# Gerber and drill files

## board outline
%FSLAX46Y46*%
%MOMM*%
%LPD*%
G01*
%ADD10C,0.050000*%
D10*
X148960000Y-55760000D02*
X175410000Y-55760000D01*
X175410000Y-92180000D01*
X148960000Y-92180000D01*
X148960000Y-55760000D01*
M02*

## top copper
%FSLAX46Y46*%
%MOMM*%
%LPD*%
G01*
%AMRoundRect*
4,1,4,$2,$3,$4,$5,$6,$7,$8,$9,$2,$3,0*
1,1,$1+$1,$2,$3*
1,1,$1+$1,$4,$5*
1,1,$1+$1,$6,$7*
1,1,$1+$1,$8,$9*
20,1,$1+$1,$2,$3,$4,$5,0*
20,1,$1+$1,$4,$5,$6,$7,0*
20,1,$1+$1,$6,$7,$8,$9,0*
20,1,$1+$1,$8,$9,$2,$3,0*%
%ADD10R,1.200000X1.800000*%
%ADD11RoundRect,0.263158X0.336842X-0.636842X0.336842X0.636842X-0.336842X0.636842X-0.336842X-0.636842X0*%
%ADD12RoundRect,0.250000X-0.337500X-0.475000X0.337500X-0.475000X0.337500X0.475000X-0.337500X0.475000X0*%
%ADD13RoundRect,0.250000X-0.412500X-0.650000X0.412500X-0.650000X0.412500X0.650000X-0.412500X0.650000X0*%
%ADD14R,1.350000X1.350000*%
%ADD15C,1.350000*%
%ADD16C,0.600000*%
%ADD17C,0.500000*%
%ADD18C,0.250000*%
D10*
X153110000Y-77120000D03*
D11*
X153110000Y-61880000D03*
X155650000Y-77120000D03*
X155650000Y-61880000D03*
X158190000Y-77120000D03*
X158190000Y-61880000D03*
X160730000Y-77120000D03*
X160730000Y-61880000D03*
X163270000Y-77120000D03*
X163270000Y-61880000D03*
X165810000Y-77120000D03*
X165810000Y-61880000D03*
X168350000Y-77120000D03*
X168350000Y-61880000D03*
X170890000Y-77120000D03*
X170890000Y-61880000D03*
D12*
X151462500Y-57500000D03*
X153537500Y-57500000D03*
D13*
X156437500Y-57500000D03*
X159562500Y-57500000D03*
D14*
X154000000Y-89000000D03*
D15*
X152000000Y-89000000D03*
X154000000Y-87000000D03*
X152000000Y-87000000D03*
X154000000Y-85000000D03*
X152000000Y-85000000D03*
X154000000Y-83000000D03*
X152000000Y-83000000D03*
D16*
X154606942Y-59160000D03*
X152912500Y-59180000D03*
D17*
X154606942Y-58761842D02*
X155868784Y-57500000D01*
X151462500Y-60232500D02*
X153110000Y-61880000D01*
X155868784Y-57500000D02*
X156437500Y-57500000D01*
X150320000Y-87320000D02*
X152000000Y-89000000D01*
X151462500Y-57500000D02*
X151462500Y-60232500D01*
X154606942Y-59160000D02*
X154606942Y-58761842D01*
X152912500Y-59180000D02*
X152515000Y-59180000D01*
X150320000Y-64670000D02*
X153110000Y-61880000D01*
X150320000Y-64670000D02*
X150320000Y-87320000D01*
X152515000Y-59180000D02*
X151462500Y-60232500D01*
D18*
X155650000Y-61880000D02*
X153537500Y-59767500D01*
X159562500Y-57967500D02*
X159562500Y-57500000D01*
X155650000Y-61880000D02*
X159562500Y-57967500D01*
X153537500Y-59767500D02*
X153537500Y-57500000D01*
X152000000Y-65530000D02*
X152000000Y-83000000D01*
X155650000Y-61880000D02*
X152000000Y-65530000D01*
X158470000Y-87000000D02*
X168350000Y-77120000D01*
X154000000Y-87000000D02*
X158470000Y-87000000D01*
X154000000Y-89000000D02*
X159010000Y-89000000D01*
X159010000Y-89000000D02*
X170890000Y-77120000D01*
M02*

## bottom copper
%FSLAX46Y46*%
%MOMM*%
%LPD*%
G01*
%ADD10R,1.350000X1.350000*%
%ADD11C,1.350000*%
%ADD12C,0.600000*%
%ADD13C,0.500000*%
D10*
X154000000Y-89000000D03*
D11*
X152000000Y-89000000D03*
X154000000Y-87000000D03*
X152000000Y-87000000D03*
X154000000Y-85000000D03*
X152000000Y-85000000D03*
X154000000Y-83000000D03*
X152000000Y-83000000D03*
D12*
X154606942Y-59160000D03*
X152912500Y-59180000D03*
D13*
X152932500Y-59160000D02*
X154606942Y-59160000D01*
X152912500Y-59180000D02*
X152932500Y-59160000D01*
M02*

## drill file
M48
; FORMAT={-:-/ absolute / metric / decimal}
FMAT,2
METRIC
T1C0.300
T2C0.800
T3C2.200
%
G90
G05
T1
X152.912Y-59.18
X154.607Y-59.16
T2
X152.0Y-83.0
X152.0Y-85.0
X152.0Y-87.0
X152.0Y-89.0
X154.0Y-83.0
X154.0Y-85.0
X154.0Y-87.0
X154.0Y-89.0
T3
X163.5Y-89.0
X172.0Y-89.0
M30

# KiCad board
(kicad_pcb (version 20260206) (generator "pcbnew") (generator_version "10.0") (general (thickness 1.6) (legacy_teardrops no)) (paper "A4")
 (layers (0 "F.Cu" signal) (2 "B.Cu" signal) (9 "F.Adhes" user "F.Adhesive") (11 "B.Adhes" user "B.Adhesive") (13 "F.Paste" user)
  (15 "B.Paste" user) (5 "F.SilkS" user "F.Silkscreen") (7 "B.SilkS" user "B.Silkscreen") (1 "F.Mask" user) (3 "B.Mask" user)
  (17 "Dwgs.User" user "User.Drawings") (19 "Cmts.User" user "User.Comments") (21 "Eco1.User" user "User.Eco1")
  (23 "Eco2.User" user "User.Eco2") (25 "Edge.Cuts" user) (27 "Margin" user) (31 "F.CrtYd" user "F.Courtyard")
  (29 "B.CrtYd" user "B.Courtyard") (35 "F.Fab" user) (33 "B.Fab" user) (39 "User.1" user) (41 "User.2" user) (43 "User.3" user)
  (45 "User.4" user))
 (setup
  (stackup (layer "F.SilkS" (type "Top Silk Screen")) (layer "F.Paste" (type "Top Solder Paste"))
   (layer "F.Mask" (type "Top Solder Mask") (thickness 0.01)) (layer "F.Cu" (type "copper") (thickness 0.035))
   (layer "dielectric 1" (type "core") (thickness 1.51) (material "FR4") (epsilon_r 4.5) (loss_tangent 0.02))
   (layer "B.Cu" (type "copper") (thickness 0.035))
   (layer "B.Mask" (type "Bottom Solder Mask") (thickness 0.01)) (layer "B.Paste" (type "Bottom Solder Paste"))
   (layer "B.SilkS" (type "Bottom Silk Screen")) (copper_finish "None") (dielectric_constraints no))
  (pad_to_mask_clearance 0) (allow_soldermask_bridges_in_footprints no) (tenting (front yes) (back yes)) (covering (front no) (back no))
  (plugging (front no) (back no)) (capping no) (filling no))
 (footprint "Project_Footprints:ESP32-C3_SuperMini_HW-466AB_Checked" (layer "F.Cu") (at 162 69.5 90)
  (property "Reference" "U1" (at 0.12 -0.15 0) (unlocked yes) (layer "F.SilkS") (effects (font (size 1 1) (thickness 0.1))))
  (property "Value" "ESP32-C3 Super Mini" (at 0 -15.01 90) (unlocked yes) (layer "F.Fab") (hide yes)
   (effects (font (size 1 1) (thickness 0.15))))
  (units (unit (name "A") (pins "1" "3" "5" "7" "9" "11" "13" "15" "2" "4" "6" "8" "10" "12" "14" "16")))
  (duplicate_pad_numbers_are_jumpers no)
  (pad "1" smd rect (at -7.62 -8.89 90) (size 1.8 1.2) (layers "F.Cu" "F.Mask" "F.Paste") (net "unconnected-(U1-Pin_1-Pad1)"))
  (pad "2" smd roundrect (at 7.62 -8.89 90) (size 1.8 1.2) (layers "F.Cu" "F.Mask" "F.Paste") (roundrect_rratio 0.2192982456) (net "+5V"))
  (pad "3" smd roundrect (at -7.62 -6.35 90) (size 1.8 1.2) (layers "F.Cu" "F.Mask" "F.Paste") (roundrect_rratio 0.2192982456)
   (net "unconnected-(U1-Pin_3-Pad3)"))
  (pad "4" smd roundrect (at 7.62 -6.35 90) (size 1.8 1.2) (layers "F.Cu" "F.Mask" "F.Paste") (roundrect_rratio 0.2192982456) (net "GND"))
  (pad "5" smd roundrect (at -7.62 -3.81 90) (size 1.8 1.2) (layers "F.Cu" "F.Mask" "F.Paste") (roundrect_rratio 0.2192982456)
   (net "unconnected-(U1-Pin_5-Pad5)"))
  (pad "6" smd roundrect (at 7.62 -3.81 90) (size 1.8 1.2) (layers "F.Cu" "F.Mask" "F.Paste") (roundrect_rratio 0.2192982456)
   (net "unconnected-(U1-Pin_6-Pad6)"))
  (pad "7" smd roundrect (at -7.62 -1.27 90) (size 1.8 1.2) (layers "F.Cu" "F.Mask" "F.Paste") (roundrect_rratio 0.2192982456)
   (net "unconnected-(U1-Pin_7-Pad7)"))
  (pad "8" smd roundrect (at 7.62 -1.27 90) (size 1.8 1.2) (layers "F.Cu" "F.Mask" "F.Paste") (roundrect_rratio 0.2192982456)
   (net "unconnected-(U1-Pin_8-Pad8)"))
  (pad "9" smd roundrect (at -7.62 1.27 90) (size 1.8 1.2) (layers "F.Cu" "F.Mask" "F.Paste") (roundrect_rratio 0.2192982456)
   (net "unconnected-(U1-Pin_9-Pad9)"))
  (pad "10" smd roundrect (at 7.62 1.27 90) (size 1.8 1.2) (layers "F.Cu" "F.Mask" "F.Paste") (roundrect_rratio 0.2192982456)
   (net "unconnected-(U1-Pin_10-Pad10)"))
  (pad "11" smd roundrect (at -7.62 3.81 90) (size 1.8 1.2) (layers "F.Cu" "F.Mask" "F.Paste") (roundrect_rratio 0.2192982456)
   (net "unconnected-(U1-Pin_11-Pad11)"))
  (pad "12" smd roundrect (at 7.62 3.81 90) (size 1.8 1.2) (layers "F.Cu" "F.Mask" "F.Paste") (roundrect_rratio 0.2192982456)
   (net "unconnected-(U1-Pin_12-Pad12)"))
  (pad "13" smd roundrect (at -7.62 6.35 90) (size 1.8 1.2) (layers "F.Cu" "F.Mask" "F.Paste") (roundrect_rratio 0.2192982456)
   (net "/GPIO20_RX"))
  (pad "14" smd roundrect (at 7.62 6.35 90) (size 1.8 1.2) (layers "F.Cu" "F.Mask" "F.Paste") (roundrect_rratio 0.2192982456)
   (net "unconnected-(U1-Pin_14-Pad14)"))
  (pad "15" smd roundrect (at -7.62 8.89 90) (size 1.8 1.2) (layers "F.Cu" "F.Mask" "F.Paste") (roundrect_rratio 0.2192982456)
   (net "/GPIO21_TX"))
  (pad "16" smd roundrect (at 7.62 8.89 90) (size 1.8 1.2) (layers "F.Cu" "F.Mask" "F.Paste") (roundrect_rratio 0.2192982456)
   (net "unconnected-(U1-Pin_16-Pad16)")))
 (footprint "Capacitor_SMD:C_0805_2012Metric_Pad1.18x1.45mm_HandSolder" (layer "F.Cu") (at 152.5 57.5)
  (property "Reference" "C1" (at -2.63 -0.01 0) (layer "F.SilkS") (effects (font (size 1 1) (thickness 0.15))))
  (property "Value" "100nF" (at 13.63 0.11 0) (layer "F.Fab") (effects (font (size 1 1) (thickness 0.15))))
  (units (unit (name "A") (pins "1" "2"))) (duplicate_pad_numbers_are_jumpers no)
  (pad "1" smd roundrect (at -1.0375 0) (size 1.175 1.45) (layers "F.Cu" "F.Mask" "F.Paste") (roundrect_rratio 0.212766) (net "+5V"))
  (pad "2" smd roundrect (at 1.0375 0) (size 1.175 1.45) (layers "F.Cu" "F.Mask" "F.Paste") (roundrect_rratio 0.212766) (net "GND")))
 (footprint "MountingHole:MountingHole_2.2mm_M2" (layer "F.Cu") (at 163.5 89)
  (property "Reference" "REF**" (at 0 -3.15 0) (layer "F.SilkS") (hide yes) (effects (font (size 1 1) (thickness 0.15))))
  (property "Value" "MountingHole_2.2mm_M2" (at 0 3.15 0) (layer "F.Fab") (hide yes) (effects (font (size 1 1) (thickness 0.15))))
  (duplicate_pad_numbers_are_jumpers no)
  (pad "" np_thru_hole circle (at 0 0) (size 2.2 2.2) (drill 2.2) (layers "*.Cu" "*.Mask")))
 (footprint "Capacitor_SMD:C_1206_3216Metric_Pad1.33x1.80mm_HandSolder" (layer "F.Cu") (at 158 57.5)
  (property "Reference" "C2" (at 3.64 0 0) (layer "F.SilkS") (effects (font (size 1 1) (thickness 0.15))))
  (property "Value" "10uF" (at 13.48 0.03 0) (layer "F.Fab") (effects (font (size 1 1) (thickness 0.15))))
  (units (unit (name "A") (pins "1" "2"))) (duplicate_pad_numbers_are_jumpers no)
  (pad "1" smd roundrect (at -1.5625 0) (size 1.325 1.8) (layers "F.Cu" "F.Mask" "F.Paste") (roundrect_rratio 0.188679) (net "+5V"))
  (pad "2" smd roundrect (at 1.5625 0) (size 1.325 1.8) (layers "F.Cu" "F.Mask" "F.Paste") (roundrect_rratio 0.188679) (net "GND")))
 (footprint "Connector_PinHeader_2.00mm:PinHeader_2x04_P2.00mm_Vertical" (layer "F.Cu") (at 154 89 180)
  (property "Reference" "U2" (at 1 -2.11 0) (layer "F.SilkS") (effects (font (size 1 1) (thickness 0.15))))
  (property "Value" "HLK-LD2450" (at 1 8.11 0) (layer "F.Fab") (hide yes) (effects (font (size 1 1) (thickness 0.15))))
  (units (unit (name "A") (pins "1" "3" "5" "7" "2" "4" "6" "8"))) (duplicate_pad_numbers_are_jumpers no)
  (pad "1" thru_hole rect (at 0 0 180) (size 1.35 1.35) (drill 0.8) (layers "*.Cu" "*.Mask") (remove_unused_layers no) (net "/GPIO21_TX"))
  (pad "2" thru_hole circle (at 2 0 180) (size 1.35 1.35) (drill 0.8) (layers "*.Cu" "*.Mask") (remove_unused_layers no) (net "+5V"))
  (pad "3" thru_hole circle (at 0 2 180) (size 1.35 1.35) (drill 0.8) (layers "*.Cu" "*.Mask") (remove_unused_layers no) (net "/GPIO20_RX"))
  (pad "4" thru_hole circle (at 2 2 180) (size 1.35 1.35) (drill 0.8) (layers "*.Cu" "*.Mask") (remove_unused_layers no)
   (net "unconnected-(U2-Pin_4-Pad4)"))
  (pad "5" thru_hole circle (at 0 4 180) (size 1.35 1.35) (drill 0.8) (layers "*.Cu" "*.Mask") (remove_unused_layers no) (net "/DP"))
  (pad "6" thru_hole circle (at 2 4 180) (size 1.35 1.35) (drill 0.8) (layers "*.Cu" "*.Mask") (remove_unused_layers no)
   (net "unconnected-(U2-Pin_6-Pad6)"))
  (pad "7" thru_hole circle (at 0 6 180) (size 1.35 1.35) (drill 0.8) (layers "*.Cu" "*.Mask") (remove_unused_layers no) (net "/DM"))
  (pad "8" thru_hole circle (at 2 6 180) (size 1.35 1.35) (drill 0.8) (layers "*.Cu" "*.Mask") (remove_unused_layers no) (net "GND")))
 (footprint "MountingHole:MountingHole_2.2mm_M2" (layer "F.Cu") (at 172 89)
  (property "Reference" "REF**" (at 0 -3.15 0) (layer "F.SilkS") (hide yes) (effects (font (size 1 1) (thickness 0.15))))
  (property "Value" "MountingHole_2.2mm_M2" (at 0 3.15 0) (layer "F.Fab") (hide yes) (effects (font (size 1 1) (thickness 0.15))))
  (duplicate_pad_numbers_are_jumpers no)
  (pad "" np_thru_hole circle (at 0 0) (size 2.2 2.2) (drill 2.2) (layers "*.Cu" "*.Mask")))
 (gr_rect (start 148.96 55.76) (end 175.41 92.18) (stroke (width 0.05) (type default)) (fill no) (layer "Edge.Cuts"))
 (segment (start 154.606942 58.761842) (end 155.868784 57.5) (width 0.5) (layer "F.Cu") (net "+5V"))
 (segment (start 151.4625 60.2325) (end 153.11 61.88) (width 0.5) (layer "F.Cu") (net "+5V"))
 (segment (start 155.868784 57.5) (end 156.4375 57.5) (width 0.5) (layer "F.Cu") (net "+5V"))
 (segment (start 150.32 87.32) (end 152 89) (width 0.5) (layer "F.Cu") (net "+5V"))
 (segment (start 151.4625 57.5) (end 151.4625 60.2325) (width 0.5) (layer "F.Cu") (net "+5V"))
 (segment (start 154.606942 59.16) (end 154.606942 58.761842) (width 0.5) (layer "F.Cu") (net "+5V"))
 (segment (start 152.9125 59.18) (end 152.515 59.18) (width 0.5) (layer "F.Cu") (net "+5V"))
 (segment (start 150.32 64.67) (end 153.11 61.88) (width 0.5) (layer "F.Cu") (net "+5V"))
 (segment (start 150.32 64.67) (end 150.32 87.32) (width 0.5) (layer "F.Cu") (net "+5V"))
 (segment (start 152.515 59.18) (end 151.4625 60.2325) (width 0.5) (layer "F.Cu") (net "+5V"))
 (via (at 154.606942 59.16) (size 0.6) (drill 0.3) (layers "F.Cu" "B.Cu") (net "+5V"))
 (via (at 152.9125 59.18) (size 0.6) (drill 0.3) (layers "F.Cu" "B.Cu") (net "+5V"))
 (segment (start 152.9325 59.16) (end 154.606942 59.16) (width 0.5) (layer "B.Cu") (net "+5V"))
 (segment (start 152.9125 59.18) (end 152.9325 59.16) (width 0.5) (layer "B.Cu") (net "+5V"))
 (segment (start 155.65 61.88) (end 153.5375 59.7675) (width 0.25) (layer "F.Cu") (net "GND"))
 (segment (start 159.5625 57.9675) (end 159.5625 57.5) (width 0.25) (layer "F.Cu") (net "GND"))
 (segment (start 155.65 61.88) (end 159.5625 57.9675) (width 0.25) (layer "F.Cu") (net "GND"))
 (segment (start 153.5375 59.7675) (end 153.5375 57.5) (width 0.25) (layer "F.Cu") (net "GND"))
 (segment (start 152 65.53) (end 152 83) (width 0.25) (layer "F.Cu") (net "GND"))
 (segment (start 155.65 61.88) (end 152 65.53) (width 0.25) (layer "F.Cu") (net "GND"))
 (segment (start 158.47 87) (end 168.35 77.12) (width 0.25) (layer "F.Cu") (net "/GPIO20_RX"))
 (segment (start 154 87) (end 158.47 87) (width 0.25) (layer "F.Cu") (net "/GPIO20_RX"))
 (segment (start 154 89) (end 159.01 89) (width 0.25) (layer "F.Cu") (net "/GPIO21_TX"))
 (segment (start 159.01 89) (end 170.89 77.12) (width 0.25) (layer "F.Cu") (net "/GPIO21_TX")))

